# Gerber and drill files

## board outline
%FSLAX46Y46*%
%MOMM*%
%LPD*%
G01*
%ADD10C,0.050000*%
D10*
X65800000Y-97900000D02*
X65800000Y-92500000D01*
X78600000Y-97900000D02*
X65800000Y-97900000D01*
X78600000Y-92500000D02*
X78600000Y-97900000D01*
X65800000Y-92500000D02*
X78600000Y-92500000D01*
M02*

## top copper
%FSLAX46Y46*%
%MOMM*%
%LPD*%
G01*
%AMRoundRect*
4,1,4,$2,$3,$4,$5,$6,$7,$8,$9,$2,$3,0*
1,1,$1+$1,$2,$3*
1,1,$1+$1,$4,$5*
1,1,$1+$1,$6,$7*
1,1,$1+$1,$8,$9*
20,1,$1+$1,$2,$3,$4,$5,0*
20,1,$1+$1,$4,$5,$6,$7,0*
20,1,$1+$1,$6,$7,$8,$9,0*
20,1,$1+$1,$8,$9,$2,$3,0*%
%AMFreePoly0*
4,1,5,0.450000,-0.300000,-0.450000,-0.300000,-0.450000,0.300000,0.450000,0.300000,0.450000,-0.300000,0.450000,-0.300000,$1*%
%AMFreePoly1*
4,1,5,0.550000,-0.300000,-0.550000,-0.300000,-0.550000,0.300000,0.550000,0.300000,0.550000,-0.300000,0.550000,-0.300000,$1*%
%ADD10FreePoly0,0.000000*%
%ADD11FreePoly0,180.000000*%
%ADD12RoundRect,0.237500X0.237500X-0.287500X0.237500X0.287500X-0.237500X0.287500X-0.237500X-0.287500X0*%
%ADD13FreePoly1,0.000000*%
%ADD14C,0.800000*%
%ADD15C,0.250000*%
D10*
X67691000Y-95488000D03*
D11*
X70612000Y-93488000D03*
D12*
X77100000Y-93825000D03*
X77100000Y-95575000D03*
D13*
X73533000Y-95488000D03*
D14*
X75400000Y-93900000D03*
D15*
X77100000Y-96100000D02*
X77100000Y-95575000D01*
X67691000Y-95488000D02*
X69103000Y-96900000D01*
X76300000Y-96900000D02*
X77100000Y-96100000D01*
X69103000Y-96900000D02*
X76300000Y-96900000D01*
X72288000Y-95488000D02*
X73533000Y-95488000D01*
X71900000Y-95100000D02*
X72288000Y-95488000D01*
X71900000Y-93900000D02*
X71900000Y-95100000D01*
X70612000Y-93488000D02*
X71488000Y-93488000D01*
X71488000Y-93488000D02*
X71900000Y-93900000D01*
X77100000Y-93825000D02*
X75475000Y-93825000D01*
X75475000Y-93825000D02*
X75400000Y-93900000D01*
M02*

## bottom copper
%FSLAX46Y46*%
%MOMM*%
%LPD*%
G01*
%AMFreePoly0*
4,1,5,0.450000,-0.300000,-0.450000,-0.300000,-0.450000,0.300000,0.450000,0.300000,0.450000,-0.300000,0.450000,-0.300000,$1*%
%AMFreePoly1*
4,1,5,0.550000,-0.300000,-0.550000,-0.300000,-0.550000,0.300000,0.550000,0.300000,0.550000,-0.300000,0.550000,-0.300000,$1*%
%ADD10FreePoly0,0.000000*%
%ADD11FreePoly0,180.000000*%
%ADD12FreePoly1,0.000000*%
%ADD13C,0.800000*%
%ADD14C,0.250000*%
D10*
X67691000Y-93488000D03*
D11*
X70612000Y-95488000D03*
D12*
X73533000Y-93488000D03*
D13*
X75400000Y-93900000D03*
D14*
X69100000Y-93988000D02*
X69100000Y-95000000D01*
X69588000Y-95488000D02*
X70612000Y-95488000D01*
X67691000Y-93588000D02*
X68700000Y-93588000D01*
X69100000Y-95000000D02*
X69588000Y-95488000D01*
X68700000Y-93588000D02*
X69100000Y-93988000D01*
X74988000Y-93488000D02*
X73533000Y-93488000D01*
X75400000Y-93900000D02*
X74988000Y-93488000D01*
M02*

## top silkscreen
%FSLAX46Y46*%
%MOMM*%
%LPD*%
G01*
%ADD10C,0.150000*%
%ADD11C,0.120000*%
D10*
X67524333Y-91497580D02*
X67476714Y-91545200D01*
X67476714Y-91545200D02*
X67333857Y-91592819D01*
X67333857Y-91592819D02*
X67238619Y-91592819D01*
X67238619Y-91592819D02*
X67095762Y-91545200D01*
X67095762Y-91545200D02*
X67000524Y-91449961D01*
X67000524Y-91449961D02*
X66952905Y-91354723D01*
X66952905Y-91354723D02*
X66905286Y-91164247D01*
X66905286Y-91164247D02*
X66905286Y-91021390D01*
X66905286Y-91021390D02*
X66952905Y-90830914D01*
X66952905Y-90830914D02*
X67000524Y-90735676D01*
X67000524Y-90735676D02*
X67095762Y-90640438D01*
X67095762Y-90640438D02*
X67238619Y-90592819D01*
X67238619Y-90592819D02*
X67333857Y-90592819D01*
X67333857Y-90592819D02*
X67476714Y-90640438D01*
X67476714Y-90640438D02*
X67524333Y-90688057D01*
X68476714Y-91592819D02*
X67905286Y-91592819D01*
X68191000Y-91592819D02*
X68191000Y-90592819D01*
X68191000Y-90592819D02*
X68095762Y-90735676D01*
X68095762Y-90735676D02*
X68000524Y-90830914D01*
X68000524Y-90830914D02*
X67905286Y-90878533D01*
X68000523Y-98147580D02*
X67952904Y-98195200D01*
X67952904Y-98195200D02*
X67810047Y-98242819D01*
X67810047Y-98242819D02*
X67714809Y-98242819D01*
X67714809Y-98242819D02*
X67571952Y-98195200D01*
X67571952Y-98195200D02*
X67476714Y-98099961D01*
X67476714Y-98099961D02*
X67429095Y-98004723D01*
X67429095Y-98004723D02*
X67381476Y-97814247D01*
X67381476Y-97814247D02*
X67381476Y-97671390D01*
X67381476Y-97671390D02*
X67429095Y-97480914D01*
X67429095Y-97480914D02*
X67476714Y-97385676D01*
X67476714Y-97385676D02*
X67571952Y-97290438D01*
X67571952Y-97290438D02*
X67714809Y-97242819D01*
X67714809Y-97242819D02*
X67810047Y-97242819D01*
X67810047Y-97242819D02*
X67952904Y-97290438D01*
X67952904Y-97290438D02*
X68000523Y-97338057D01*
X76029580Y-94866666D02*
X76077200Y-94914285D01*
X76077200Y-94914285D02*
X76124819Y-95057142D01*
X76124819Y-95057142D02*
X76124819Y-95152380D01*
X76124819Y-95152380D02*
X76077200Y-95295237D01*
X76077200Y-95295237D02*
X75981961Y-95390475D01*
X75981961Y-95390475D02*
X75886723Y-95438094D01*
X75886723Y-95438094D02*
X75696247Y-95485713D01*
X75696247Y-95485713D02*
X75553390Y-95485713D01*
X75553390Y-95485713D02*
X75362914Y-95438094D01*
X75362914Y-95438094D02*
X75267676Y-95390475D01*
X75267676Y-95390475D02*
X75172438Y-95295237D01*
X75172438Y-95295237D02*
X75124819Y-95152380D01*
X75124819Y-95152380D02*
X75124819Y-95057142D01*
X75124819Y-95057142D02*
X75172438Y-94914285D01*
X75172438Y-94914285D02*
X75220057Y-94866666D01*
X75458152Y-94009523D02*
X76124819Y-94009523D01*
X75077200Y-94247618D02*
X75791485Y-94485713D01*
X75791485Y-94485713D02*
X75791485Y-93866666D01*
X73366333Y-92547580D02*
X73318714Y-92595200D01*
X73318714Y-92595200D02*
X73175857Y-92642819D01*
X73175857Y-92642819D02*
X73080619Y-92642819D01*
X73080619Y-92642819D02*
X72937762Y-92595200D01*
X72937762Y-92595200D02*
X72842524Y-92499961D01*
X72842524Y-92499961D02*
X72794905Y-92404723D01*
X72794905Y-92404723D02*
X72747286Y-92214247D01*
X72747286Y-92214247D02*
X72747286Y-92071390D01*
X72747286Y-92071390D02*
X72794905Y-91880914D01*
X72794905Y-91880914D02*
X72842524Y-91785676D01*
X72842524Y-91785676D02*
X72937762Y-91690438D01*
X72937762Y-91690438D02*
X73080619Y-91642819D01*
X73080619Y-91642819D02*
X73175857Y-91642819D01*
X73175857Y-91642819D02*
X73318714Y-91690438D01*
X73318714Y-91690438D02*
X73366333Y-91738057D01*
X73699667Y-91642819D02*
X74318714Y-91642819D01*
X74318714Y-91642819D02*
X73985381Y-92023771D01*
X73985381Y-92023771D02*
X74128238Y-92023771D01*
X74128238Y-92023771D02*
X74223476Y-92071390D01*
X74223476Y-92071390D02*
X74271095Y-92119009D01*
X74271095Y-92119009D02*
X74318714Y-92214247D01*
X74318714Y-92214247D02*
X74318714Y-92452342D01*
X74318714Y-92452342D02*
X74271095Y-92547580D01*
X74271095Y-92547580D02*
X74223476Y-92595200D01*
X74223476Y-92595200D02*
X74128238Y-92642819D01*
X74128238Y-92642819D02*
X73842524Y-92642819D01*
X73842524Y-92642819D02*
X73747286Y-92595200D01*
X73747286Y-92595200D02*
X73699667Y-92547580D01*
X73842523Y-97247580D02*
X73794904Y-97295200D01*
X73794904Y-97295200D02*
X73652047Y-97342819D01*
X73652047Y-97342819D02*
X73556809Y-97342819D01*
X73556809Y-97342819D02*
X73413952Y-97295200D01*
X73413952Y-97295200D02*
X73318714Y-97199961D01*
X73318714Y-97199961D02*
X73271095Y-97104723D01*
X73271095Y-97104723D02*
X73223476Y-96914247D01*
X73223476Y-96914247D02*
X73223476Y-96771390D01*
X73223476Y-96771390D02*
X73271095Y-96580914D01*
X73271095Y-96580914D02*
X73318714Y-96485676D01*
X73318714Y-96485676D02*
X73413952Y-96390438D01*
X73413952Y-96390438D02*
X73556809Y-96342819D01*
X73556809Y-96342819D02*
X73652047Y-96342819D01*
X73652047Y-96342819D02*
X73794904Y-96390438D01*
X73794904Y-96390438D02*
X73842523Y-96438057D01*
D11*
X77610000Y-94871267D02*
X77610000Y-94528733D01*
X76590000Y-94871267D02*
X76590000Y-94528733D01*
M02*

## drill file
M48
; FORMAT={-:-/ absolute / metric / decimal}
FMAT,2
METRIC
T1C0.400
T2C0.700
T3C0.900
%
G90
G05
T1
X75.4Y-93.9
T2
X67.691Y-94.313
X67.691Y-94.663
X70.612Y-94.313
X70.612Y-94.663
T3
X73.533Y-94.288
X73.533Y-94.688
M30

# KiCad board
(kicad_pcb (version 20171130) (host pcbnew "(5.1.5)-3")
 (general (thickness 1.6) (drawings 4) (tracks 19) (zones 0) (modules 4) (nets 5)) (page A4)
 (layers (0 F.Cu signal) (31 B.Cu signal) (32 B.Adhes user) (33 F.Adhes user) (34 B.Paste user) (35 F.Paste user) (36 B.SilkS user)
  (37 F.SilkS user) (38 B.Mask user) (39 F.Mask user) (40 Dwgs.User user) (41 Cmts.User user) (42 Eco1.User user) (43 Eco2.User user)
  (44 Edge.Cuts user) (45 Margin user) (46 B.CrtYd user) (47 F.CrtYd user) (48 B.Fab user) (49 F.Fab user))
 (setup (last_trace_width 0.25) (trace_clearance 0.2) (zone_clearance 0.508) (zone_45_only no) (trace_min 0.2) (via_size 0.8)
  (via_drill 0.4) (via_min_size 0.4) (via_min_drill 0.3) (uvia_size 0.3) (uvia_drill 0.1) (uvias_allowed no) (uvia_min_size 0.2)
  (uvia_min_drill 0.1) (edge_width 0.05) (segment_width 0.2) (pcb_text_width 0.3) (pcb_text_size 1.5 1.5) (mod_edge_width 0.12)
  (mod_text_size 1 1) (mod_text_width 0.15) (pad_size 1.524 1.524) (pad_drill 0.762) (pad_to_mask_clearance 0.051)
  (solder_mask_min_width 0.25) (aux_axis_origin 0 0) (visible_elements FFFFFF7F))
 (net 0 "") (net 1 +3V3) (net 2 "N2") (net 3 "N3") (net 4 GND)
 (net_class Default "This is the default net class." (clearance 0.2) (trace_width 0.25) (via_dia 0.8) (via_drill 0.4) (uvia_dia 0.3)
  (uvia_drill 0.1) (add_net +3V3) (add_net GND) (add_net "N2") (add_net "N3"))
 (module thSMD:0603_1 (layer F.Cu) (at 67.691 94.488) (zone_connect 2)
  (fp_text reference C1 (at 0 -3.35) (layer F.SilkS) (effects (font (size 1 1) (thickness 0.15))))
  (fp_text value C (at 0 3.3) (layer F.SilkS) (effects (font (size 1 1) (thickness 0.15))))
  (pad 1 smd custom (at 0 1) (size 0.9 0.6) (layers F.Cu F.Mask) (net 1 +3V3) (zone_connect 0) (options (clearance outline) (anchor rect))
   (primitives))
  (pad 2 smd custom (at 0 -1) (size 0.9 0.6) (layers B.Cu B.Mask) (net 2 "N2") (zone_connect 0) (options (clearance outline) (anchor rect))
   (primitives))
  (pad "" np_thru_hole circle (at 0 0.175) (size 0.7 0.7) (drill 0.7) (layers *.Cu) (zone_connect 0) (thermal_width 0.6) (thermal_gap 0.1))
  (pad "" np_thru_hole circle (at 0 -0.175) (size 0.7 0.7) (drill 0.7) (layers *.Cu) (zone_connect 0)))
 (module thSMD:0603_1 (layer B.Cu) (at 70.612 94.488 180) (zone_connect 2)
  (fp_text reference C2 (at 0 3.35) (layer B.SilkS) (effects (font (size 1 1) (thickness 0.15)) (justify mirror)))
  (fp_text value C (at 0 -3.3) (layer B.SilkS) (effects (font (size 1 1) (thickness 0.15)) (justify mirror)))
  (pad 1 smd custom (at 0 -1 180) (size 0.9 0.6) (layers B.Cu B.Mask) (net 2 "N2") (zone_connect 0)
   (options (clearance outline) (anchor rect)) (primitives))
  (pad 2 smd custom (at 0 1 180) (size 0.9 0.6) (layers F.Cu F.Mask) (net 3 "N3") (zone_connect 0)
   (options (clearance outline) (anchor rect)) (primitives))
  (pad "" np_thru_hole circle (at 0 -0.175 180) (size 0.7 0.7) (drill 0.7) (layers *.Cu) (zone_connect 0) (thermal_width 0.6)
   (thermal_gap 0.1))
  (pad "" np_thru_hole circle (at 0 0.175 180) (size 0.7 0.7) (drill 0.7) (layers *.Cu) (zone_connect 0)))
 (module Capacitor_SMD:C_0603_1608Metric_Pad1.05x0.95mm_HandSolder (layer F.Cu) (at 77.1 94.7 90)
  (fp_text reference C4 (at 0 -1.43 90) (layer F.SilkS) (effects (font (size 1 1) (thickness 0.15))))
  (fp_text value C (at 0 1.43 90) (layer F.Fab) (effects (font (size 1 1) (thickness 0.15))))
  (fp_line (start -0.171267 0.51) (end 0.171267 0.51) (layer F.SilkS) (width 0.12))
  (fp_line (start -0.171267 -0.51) (end 0.171267 -0.51) (layer F.SilkS) (width 0.12))
  (pad 2 smd roundrect (at 0.875 0 90) (size 1.05 0.95) (layers F.Cu F.Paste F.Mask) (roundrect_rratio 0.25) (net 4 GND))
  (pad 1 smd roundrect (at -0.875 0 90) (size 1.05 0.95) (layers F.Cu F.Paste F.Mask) (roundrect_rratio 0.25) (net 1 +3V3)))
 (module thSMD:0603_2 (layer F.Cu) (at 73.533 94.488) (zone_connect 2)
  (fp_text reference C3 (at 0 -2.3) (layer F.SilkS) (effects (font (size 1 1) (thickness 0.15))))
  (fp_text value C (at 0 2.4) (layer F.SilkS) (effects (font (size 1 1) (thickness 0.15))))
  (pad 1 smd custom (at 0 1) (size 1.1 0.6) (layers F.Cu F.Mask) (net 3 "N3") (zone_connect 0) (options (clearance outline) (anchor rect))
   (primitives))
  (pad 2 smd custom (at 0 -1) (size 1.1 0.6) (layers B.Cu B.Mask) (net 4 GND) (zone_connect 0) (options (clearance outline) (anchor rect))
   (primitives))
  (pad "" np_thru_hole circle (at 0 0.2) (size 0.9 0.9) (drill 0.9) (layers *.Cu) (zone_connect 0) (thermal_width 0.6) (thermal_gap 0.1))
  (pad "" np_thru_hole circle (at 0 -0.2) (size 0.9 0.9) (drill 0.9) (layers *.Cu) (zone_connect 0)))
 (gr_line (start 65.8 97.9) (end 65.8 92.5) (layer Edge.Cuts) (width 0.05))
 (gr_line (start 78.6 97.9) (end 65.8 97.9) (layer Edge.Cuts) (width 0.05))
 (gr_line (start 78.6 92.5) (end 78.6 97.9) (layer Edge.Cuts) (width 0.05))
 (gr_line (start 65.8 92.5) (end 78.6 92.5) (layer Edge.Cuts) (width 0.05))
 (segment (start 77.1 96.1) (end 77.1 95.575) (width 0.25) (layer F.Cu) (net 1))
 (segment (start 67.691 95.488) (end 69.103 96.9) (width 0.25) (layer F.Cu) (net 1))
 (segment (start 76.3 96.9) (end 77.1 96.1) (width 0.25) (layer F.Cu) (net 1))
 (segment (start 69.103 96.9) (end 76.3 96.9) (width 0.25) (layer F.Cu) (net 1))
 (segment (start 69.1 93.988) (end 69.1 95) (width 0.25) (layer B.Cu) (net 2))
 (segment (start 69.588 95.488) (end 70.612 95.488) (width 0.25) (layer B.Cu) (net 2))
 (segment (start 67.691 93.588) (end 68.7 93.588) (width 0.25) (layer B.Cu) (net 2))
 (segment (start 69.1 95) (end 69.588 95.488) (width 0.25) (layer B.Cu) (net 2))
 (segment (start 68.7 93.588) (end 69.1 93.988) (width 0.25) (layer B.Cu) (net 2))
 (segment (start 72.288 95.488) (end 73.533 95.488) (width 0.25) (layer F.Cu) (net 3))
 (segment (start 71.9 95.1) (end 72.288 95.488) (width 0.25) (layer F.Cu) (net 3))
 (segment (start 71.9 93.9) (end 71.9 95.1) (width 0.25) (layer F.Cu) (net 3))
 (segment (start 70.612 93.488) (end 71.488 93.488) (width 0.25) (layer F.Cu) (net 3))
 (segment (start 71.488 93.488) (end 71.9 93.9) (width 0.25) (layer F.Cu) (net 3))
 (via (at 75.4 93.9) (size 0.8) (drill 0.4) (layers F.Cu B.Cu) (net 4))
 (segment (start 77.1 93.825) (end 75.475 93.825) (width 0.25) (layer F.Cu) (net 4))
 (segment (start 75.475 93.825) (end 75.4 93.9) (width 0.25) (layer F.Cu) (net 4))
 (segment (start 74.988 93.488) (end 73.533 93.488) (width 0.25) (layer B.Cu) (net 4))
 (segment (start 75.4 93.9) (end 74.988 93.488) (width 0.25) (layer B.Cu) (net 4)))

